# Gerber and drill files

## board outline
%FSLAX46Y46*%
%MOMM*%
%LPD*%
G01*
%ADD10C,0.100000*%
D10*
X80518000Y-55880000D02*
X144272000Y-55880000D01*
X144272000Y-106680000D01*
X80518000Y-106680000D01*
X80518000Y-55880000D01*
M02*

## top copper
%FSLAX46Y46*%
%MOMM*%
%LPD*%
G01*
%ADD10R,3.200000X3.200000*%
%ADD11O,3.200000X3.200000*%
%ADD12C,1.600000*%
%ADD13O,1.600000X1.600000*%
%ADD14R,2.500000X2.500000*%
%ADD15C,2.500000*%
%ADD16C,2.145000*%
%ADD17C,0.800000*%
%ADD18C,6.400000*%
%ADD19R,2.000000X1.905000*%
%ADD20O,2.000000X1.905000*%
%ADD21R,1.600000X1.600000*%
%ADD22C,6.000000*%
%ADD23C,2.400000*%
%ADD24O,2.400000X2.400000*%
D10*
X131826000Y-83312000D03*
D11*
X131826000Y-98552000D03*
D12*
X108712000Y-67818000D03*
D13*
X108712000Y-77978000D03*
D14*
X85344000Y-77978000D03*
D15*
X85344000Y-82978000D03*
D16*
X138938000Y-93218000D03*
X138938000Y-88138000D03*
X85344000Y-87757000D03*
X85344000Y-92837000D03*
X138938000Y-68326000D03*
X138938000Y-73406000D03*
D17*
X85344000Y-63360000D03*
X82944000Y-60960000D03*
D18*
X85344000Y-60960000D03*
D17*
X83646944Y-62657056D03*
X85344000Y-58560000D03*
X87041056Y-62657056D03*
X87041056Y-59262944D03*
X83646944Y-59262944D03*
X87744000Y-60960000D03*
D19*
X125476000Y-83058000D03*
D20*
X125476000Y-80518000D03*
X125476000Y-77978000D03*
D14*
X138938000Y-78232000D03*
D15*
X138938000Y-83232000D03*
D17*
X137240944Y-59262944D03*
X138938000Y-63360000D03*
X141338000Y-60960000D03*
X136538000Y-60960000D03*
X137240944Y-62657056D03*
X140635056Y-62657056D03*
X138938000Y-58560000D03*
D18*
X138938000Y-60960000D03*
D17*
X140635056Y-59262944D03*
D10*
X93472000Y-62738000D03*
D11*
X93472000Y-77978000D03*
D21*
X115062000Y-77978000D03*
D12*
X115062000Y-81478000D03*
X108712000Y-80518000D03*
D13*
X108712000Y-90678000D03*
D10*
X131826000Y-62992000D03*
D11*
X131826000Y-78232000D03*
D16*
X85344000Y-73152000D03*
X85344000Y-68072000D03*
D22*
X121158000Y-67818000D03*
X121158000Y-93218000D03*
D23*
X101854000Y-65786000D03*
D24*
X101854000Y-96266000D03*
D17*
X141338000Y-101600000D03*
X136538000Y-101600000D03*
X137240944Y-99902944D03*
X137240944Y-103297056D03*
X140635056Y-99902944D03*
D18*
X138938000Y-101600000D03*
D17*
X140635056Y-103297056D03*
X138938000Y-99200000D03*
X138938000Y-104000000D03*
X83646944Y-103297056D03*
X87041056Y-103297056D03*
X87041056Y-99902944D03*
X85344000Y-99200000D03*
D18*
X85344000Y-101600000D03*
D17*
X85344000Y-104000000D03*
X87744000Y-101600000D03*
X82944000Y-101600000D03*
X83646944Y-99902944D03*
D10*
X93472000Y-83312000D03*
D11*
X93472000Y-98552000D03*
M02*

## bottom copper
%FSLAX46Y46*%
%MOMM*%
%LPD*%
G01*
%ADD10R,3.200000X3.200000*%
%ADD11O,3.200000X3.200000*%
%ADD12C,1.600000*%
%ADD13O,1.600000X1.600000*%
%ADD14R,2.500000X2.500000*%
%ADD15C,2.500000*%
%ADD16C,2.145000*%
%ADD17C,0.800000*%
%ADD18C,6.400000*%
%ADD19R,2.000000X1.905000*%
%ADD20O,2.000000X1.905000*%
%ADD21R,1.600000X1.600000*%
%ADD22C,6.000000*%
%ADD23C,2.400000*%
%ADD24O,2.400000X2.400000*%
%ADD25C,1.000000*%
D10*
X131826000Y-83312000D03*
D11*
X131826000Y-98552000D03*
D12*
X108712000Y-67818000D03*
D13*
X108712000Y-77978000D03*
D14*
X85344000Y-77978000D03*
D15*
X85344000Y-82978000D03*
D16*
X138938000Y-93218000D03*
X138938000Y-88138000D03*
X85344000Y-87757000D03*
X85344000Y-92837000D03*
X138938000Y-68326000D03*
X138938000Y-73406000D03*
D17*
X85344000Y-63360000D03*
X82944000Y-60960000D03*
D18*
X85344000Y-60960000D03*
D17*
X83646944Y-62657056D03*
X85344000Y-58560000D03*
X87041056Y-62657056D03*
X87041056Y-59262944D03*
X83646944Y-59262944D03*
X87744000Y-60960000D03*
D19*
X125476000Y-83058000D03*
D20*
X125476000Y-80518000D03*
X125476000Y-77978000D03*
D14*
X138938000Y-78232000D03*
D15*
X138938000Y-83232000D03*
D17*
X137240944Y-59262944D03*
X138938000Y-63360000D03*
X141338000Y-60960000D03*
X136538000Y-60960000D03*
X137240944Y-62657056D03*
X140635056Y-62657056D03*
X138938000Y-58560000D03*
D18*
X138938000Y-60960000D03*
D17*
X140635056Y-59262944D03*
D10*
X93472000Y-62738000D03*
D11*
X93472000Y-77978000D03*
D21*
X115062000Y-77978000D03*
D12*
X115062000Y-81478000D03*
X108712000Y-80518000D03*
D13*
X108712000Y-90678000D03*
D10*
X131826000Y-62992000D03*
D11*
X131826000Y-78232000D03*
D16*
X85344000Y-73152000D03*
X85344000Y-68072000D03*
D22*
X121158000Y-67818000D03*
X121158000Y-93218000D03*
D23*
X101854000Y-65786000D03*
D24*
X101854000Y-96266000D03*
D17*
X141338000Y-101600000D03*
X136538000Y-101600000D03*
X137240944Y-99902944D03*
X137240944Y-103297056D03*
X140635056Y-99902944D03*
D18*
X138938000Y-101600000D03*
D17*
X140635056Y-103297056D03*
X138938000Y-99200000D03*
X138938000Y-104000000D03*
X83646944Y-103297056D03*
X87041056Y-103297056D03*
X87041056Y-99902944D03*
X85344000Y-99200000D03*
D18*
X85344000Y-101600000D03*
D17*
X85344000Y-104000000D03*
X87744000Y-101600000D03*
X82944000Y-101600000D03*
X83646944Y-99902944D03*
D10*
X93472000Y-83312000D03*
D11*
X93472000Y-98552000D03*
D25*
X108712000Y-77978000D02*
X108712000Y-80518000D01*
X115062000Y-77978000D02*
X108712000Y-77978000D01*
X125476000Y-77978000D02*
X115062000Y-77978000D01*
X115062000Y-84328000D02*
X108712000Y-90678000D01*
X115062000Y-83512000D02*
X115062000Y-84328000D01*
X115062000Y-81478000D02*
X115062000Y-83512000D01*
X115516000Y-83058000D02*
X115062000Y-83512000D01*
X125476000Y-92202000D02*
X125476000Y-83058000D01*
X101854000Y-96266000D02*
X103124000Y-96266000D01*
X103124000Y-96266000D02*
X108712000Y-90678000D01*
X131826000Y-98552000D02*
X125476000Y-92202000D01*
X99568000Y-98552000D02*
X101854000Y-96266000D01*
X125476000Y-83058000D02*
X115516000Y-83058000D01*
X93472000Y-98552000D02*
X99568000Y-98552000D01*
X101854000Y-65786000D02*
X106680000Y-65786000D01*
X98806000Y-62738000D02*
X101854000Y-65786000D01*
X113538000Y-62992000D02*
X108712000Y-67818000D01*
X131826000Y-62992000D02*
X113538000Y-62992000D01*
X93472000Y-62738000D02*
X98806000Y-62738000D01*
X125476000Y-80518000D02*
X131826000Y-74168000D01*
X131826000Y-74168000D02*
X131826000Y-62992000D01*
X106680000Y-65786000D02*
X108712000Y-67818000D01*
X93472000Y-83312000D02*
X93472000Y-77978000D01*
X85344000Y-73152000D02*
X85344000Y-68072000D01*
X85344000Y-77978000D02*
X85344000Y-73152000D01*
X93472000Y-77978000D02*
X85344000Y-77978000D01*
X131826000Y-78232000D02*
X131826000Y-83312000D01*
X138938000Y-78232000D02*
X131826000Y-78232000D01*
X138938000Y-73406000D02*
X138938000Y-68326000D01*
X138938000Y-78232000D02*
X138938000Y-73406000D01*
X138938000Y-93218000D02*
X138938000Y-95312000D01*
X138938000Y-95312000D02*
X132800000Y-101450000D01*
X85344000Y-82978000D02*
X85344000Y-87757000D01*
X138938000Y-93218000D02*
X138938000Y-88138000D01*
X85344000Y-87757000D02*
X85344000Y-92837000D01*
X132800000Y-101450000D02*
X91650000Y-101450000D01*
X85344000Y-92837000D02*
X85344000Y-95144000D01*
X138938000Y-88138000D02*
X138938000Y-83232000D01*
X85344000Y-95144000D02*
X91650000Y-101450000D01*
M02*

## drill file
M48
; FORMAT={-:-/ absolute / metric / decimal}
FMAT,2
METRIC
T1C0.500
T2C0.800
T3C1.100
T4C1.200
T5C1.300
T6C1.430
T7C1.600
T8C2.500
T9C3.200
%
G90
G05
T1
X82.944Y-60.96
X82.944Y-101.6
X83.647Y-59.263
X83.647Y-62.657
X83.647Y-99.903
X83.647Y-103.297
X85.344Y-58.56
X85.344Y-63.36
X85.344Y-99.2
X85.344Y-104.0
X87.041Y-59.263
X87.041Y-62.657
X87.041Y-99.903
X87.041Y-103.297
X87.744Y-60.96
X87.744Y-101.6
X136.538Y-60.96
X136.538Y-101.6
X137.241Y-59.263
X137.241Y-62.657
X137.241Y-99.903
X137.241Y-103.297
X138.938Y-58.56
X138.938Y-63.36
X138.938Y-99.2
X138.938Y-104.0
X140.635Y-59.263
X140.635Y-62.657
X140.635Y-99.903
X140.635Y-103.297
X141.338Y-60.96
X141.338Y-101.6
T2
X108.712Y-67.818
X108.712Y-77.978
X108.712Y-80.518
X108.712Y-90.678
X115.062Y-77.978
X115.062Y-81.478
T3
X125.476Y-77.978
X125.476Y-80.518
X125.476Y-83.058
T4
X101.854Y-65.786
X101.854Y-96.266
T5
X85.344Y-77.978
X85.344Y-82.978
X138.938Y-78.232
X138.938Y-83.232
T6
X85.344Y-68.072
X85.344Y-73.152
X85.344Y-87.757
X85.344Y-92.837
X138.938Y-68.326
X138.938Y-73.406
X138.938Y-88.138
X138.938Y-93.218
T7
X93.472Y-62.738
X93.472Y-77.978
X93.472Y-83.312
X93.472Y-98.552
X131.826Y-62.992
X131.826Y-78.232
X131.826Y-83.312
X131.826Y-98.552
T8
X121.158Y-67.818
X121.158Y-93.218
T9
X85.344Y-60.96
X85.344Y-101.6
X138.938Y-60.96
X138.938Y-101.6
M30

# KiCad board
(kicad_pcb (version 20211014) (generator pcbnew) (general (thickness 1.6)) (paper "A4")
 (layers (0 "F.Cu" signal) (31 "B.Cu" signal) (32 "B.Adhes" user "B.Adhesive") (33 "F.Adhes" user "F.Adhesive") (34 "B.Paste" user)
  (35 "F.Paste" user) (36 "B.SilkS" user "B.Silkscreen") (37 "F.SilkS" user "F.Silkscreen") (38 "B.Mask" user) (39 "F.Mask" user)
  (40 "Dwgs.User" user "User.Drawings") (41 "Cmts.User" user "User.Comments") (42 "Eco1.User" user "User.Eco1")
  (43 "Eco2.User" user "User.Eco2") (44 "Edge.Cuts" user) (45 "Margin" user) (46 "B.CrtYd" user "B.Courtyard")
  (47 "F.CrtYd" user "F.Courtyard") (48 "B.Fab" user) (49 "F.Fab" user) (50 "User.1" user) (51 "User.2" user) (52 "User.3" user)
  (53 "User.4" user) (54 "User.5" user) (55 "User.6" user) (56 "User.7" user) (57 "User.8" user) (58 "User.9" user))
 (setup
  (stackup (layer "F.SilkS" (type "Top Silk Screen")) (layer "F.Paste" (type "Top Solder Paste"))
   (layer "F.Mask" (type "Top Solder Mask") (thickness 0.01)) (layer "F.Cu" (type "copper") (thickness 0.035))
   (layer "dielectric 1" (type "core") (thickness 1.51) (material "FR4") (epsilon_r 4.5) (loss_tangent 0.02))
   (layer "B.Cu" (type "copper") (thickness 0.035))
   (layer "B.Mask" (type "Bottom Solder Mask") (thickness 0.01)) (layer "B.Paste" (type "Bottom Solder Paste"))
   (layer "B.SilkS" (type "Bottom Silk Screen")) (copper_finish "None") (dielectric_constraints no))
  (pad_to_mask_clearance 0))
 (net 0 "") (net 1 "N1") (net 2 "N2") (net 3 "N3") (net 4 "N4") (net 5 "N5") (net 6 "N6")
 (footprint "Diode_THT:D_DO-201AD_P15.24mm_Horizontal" (layer "F.Cu") (at 131.826 83.312 -90)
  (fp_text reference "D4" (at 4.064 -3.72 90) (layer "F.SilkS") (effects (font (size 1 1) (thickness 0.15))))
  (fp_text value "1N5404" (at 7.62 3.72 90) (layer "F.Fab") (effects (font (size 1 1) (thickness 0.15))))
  (pad "1" thru_hole rect (at 0 0 270) (size 3.2 3.2) (drill 1.6) (layers *.Cu *.Mask) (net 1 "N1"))
  (pad "2" thru_hole oval (at 15.24 0 270) (size 3.2 3.2) (drill 1.6) (layers *.Cu *.Mask) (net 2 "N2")))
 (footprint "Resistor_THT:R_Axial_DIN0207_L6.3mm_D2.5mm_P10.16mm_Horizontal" (layer "F.Cu") (at 108.712 67.818 -90)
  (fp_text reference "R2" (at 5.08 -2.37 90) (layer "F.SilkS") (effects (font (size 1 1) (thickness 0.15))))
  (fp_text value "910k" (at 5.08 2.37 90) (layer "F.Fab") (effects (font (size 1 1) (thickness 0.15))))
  (pad "1" thru_hole circle (at 0 0 270) (size 1.6 1.6) (drill 0.8) (layers *.Cu *.Mask) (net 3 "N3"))
  (pad "2" thru_hole oval (at 10.16 0 270) (size 1.6 1.6) (drill 0.8) (layers *.Cu *.Mask) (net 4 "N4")))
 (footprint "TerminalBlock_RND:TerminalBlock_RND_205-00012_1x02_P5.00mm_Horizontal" (layer "F.Cu") (at 85.344 77.978 -90)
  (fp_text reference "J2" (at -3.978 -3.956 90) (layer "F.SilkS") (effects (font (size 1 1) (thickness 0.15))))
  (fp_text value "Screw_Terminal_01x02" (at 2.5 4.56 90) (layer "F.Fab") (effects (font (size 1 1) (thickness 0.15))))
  (pad "1" thru_hole rect (at 0 0 270) (size 2.5 2.5) (drill 1.3) (layers *.Cu *.Mask) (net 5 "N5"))
  (pad "2" thru_hole circle (at 5 0 270) (size 2.5 2.5) (drill 1.3) (layers *.Cu *.Mask) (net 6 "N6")))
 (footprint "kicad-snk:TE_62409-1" (layer "F.Cu") (at 138.938 90.678 90)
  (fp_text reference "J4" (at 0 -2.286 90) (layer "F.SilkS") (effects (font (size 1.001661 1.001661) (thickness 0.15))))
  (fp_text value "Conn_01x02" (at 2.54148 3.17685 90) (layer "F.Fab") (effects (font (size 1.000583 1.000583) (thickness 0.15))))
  (pad "1" thru_hole circle (at -2.54 0 90) (size 2.145 2.145) (drill 1.43) (layers *.Cu *.Mask) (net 6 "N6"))
  (pad "2" thru_hole circle (at 2.54 0 90) (size 2.145 2.145) (drill 1.43) (layers *.Cu *.Mask) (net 6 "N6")))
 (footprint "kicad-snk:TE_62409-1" (layer "F.Cu") (at 85.344 90.297 -90)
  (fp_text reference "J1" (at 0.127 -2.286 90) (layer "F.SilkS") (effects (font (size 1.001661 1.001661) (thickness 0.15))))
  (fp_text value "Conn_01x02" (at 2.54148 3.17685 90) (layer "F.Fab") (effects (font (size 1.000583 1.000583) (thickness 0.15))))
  (pad "1" thru_hole circle (at -2.54 0 270) (size 2.145 2.145) (drill 1.43) (layers *.Cu *.Mask) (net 6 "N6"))
  (pad "2" thru_hole circle (at 2.54 0 270) (size 2.145 2.145) (drill 1.43) (layers *.Cu *.Mask) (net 6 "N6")))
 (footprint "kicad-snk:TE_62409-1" (layer "F.Cu") (at 138.938 70.866 -90)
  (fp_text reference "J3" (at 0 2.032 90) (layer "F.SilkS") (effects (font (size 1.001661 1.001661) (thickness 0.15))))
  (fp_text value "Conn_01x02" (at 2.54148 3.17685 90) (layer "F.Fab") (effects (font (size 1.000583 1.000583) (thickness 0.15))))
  (pad "1" thru_hole circle (at -2.54 0 270) (size 2.145 2.145) (drill 1.43) (layers *.Cu *.Mask) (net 1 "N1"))
  (pad "2" thru_hole circle (at 2.54 0 270) (size 2.145 2.145) (drill 1.43) (layers *.Cu *.Mask) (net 1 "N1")))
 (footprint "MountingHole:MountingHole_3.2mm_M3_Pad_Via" (layer "F.Cu") (at 85.344 60.96)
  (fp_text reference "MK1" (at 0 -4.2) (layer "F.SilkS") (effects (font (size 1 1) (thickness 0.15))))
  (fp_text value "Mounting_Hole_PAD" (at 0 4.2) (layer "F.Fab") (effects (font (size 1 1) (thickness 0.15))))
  (pad "1" thru_hole circle (at 0 2.4) (size 0.8 0.8) (drill 0.5) (layers *.Cu *.Mask))
  (pad "1" thru_hole circle (at -2.4 0) (size 0.8 0.8) (drill 0.5) (layers *.Cu *.Mask))
  (pad "1" thru_hole circle (at 0 0) (size 6.4 6.4) (drill 3.2) (layers *.Cu *.Mask))
  (pad "1" thru_hole circle (at -1.697056 1.697056) (size 0.8 0.8) (drill 0.5) (layers *.Cu *.Mask))
  (pad "1" thru_hole circle (at 0 -2.4) (size 0.8 0.8) (drill 0.5) (layers *.Cu *.Mask))
  (pad "1" thru_hole circle (at 1.697056 1.697056) (size 0.8 0.8) (drill 0.5) (layers *.Cu *.Mask))
  (pad "1" thru_hole circle (at 1.697056 -1.697056) (size 0.8 0.8) (drill 0.5) (layers *.Cu *.Mask))
  (pad "1" thru_hole circle (at -1.697056 -1.697056) (size 0.8 0.8) (drill 0.5) (layers *.Cu *.Mask))
  (pad "1" thru_hole circle (at 2.4 0) (size 0.8 0.8) (drill 0.5) (layers *.Cu *.Mask)))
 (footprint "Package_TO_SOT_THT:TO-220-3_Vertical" (layer "F.Cu") (at 125.476 83.058 90)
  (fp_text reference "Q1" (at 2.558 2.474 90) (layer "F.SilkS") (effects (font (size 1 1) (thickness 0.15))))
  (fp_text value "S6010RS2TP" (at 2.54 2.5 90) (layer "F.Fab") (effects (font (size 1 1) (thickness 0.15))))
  (pad "1" thru_hole rect (at 0 0 90) (size 1.905 2) (drill 1.1) (layers *.Cu *.Mask) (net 2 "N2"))
  (pad "2" thru_hole oval (at 2.54 0 90) (size 1.905 2) (drill 1.1) (layers *.Cu *.Mask) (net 3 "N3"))
  (pad "3" thru_hole oval (at 5.08 0 90) (size 1.905 2) (drill 1.1) (layers *.Cu *.Mask) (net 4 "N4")))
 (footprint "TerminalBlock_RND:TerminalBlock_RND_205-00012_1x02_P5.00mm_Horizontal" (layer "F.Cu") (at 138.938 78.232 -90)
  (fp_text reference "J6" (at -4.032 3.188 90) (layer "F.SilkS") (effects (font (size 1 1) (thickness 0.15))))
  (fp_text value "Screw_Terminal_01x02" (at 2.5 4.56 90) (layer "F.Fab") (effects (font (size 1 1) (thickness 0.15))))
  (pad "1" thru_hole rect (at 0 0 270) (size 2.5 2.5) (drill 1.3) (layers *.Cu *.Mask) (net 1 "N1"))
  (pad "2" thru_hole circle (at 5 0 270) (size 2.5 2.5) (drill 1.3) (layers *.Cu *.Mask) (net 6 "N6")))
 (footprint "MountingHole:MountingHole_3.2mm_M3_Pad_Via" (layer "F.Cu") (at 138.938 60.96)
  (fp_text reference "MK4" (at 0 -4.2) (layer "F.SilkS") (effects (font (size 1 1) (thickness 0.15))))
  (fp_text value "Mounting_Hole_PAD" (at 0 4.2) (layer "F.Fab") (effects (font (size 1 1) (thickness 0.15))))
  (pad "1" thru_hole circle (at -1.697056 -1.697056) (size 0.8 0.8) (drill 0.5) (layers *.Cu *.Mask))
  (pad "1" thru_hole circle (at 0 2.4) (size 0.8 0.8) (drill 0.5) (layers *.Cu *.Mask))
  (pad "1" thru_hole circle (at 2.4 0) (size 0.8 0.8) (drill 0.5) (layers *.Cu *.Mask))
  (pad "1" thru_hole circle (at -2.4 0) (size 0.8 0.8) (drill 0.5) (layers *.Cu *.Mask))
  (pad "1" thru_hole circle (at -1.697056 1.697056) (size 0.8 0.8) (drill 0.5) (layers *.Cu *.Mask))
  (pad "1" thru_hole circle (at 1.697056 1.697056) (size 0.8 0.8) (drill 0.5) (layers *.Cu *.Mask))
  (pad "1" thru_hole circle (at 0 -2.4) (size 0.8 0.8) (drill 0.5) (layers *.Cu *.Mask))
  (pad "1" thru_hole circle (at 0 0) (size 6.4 6.4) (drill 3.2) (layers *.Cu *.Mask))
  (pad "1" thru_hole circle (at 1.697056 -1.697056) (size 0.8 0.8) (drill 0.5) (layers *.Cu *.Mask)))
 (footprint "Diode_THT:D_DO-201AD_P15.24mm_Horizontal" (layer "F.Cu") (at 93.472 62.738 -90)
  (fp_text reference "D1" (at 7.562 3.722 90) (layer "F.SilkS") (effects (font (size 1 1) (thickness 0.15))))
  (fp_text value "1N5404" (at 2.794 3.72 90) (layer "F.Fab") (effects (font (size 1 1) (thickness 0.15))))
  (pad "1" thru_hole rect (at 0 0 270) (size 3.2 3.2) (drill 1.6) (layers *.Cu *.Mask) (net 3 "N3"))
  (pad "2" thru_hole oval (at 15.24 0 270) (size 3.2 3.2) (drill 1.6) (layers *.Cu *.Mask) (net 5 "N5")))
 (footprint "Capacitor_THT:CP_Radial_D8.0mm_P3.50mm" (layer "F.Cu") (at 115.062 77.978 -90)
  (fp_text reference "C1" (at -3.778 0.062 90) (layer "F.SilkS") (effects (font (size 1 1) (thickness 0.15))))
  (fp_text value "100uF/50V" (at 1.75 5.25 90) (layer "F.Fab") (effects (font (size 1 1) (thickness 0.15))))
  (pad "1" thru_hole rect (at 0 0 270) (size 1.6 1.6) (drill 0.8) (layers *.Cu *.Mask) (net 4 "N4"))
  (pad "2" thru_hole circle (at 3.5 0 270) (size 1.6 1.6) (drill 0.8) (layers *.Cu *.Mask) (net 2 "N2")))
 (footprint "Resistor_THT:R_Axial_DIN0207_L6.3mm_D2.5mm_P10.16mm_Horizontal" (layer "F.Cu") (at 108.712 80.518 -90)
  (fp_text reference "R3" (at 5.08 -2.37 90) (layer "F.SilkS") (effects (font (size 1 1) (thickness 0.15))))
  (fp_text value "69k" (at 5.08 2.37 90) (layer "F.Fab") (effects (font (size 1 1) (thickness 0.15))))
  (pad "1" thru_hole circle (at 0 0 270) (size 1.6 1.6) (drill 0.8) (layers *.Cu *.Mask) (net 4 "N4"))
  (pad "2" thru_hole oval (at 10.16 0 270) (size 1.6 1.6) (drill 0.8) (layers *.Cu *.Mask) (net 2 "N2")))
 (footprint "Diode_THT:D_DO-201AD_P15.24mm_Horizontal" (layer "F.Cu") (at 131.826 62.992 -90)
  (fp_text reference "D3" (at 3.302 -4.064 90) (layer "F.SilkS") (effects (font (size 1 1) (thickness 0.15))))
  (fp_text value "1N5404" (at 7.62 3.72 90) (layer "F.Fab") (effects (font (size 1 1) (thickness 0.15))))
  (pad "1" thru_hole rect (at 0 0 270) (size 3.2 3.2) (drill 1.6) (layers *.Cu *.Mask) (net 3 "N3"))
  (pad "2" thru_hole oval (at 15.24 0 270) (size 3.2 3.2) (drill 1.6) (layers *.Cu *.Mask) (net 1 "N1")))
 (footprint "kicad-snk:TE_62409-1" (layer "F.Cu") (at 85.344 70.612 90)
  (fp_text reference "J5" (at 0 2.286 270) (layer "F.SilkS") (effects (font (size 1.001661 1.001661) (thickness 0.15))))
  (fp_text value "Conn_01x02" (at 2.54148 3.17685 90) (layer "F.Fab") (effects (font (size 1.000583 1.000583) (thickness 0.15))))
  (pad "1" thru_hole circle (at -2.54 0 90) (size 2.145 2.145) (drill 1.43) (layers *.Cu *.Mask) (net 5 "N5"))
  (pad "2" thru_hole circle (at 2.54 0 90) (size 2.145 2.145) (drill 1.43) (layers *.Cu *.Mask) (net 5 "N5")))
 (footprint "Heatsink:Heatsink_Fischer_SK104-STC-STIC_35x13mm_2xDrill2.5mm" (layer "F.Cu") (at 121.158 80.518 90)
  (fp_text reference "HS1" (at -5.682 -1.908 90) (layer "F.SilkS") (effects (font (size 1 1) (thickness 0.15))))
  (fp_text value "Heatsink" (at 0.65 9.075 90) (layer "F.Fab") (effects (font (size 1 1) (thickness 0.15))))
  (pad "1" thru_hole circle (at 12.7 0 90) (size 6 6) (drill 2.5) (layers *.Cu *.Mask))
  (pad "1" thru_hole circle (at -12.7 0 270) (size 6 6) (drill 2.5) (layers *.Cu *.Mask)))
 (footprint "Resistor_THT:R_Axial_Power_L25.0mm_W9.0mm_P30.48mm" (layer "F.Cu") (at 101.854 65.786 -90)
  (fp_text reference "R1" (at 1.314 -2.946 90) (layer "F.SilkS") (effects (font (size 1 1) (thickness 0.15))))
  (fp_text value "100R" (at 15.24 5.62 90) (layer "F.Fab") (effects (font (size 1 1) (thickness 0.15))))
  (pad "1" thru_hole circle (at 0 0 270) (size 2.4 2.4) (drill 1.2) (layers *.Cu *.Mask) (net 3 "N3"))
  (pad "2" thru_hole oval (at 30.48 0 270) (size 2.4 2.4) (drill 1.2) (layers *.Cu *.Mask) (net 2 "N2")))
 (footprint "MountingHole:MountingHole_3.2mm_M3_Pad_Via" (layer "F.Cu") (at 138.938 101.6)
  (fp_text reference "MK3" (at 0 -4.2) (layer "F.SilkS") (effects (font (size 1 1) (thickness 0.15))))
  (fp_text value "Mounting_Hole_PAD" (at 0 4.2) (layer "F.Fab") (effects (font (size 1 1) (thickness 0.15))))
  (pad "1" thru_hole circle (at 2.4 0) (size 0.8 0.8) (drill 0.5) (layers *.Cu *.Mask))
  (pad "1" thru_hole circle (at -2.4 0) (size 0.8 0.8) (drill 0.5) (layers *.Cu *.Mask))
  (pad "1" thru_hole circle (at -1.697056 -1.697056) (size 0.8 0.8) (drill 0.5) (layers *.Cu *.Mask))
  (pad "1" thru_hole circle (at -1.697056 1.697056) (size 0.8 0.8) (drill 0.5) (layers *.Cu *.Mask))
  (pad "1" thru_hole circle (at 1.697056 -1.697056) (size 0.8 0.8) (drill 0.5) (layers *.Cu *.Mask))
  (pad "1" thru_hole circle (at 0 0) (size 6.4 6.4) (drill 3.2) (layers *.Cu *.Mask))
  (pad "1" thru_hole circle (at 1.697056 1.697056) (size 0.8 0.8) (drill 0.5) (layers *.Cu *.Mask))
  (pad "1" thru_hole circle (at 0 -2.4) (size 0.8 0.8) (drill 0.5) (layers *.Cu *.Mask))
  (pad "1" thru_hole circle (at 0 2.4) (size 0.8 0.8) (drill 0.5) (layers *.Cu *.Mask)))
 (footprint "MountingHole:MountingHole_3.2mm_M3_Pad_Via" (layer "F.Cu") (at 85.344 101.6)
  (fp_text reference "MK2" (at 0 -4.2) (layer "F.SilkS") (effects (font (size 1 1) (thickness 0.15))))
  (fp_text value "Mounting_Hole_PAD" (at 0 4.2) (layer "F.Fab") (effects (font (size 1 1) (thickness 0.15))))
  (pad "1" thru_hole circle (at -1.697056 1.697056) (size 0.8 0.8) (drill 0.5) (layers *.Cu *.Mask))
  (pad "1" thru_hole circle (at 1.697056 1.697056) (size 0.8 0.8) (drill 0.5) (layers *.Cu *.Mask))
  (pad "1" thru_hole circle (at 1.697056 -1.697056) (size 0.8 0.8) (drill 0.5) (layers *.Cu *.Mask))
  (pad "1" thru_hole circle (at 0 -2.4) (size 0.8 0.8) (drill 0.5) (layers *.Cu *.Mask))
  (pad "1" thru_hole circle (at 0 0) (size 6.4 6.4) (drill 3.2) (layers *.Cu *.Mask))
  (pad "1" thru_hole circle (at 0 2.4) (size 0.8 0.8) (drill 0.5) (layers *.Cu *.Mask))
  (pad "1" thru_hole circle (at 2.4 0) (size 0.8 0.8) (drill 0.5) (layers *.Cu *.Mask))
  (pad "1" thru_hole circle (at -2.4 0) (size 0.8 0.8) (drill 0.5) (layers *.Cu *.Mask))
  (pad "1" thru_hole circle (at -1.697056 -1.697056) (size 0.8 0.8) (drill 0.5) (layers *.Cu *.Mask)))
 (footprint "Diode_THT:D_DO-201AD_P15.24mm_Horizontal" (layer "F.Cu") (at 93.472 83.312 -90)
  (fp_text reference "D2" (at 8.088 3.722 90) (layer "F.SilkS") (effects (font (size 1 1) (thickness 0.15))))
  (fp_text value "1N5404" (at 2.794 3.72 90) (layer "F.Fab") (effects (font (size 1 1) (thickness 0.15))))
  (pad "1" thru_hole rect (at 0 0 270) (size 3.2 3.2) (drill 1.6) (layers *.Cu *.Mask) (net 5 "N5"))
  (pad "2" thru_hole oval (at 15.24 0 270) (size 3.2 3.2) (drill 1.6) (layers *.Cu *.Mask) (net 2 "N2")))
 (gr_rect (start 80.518 55.88) (end 144.272 106.68) (layer "Edge.Cuts") (width 0.1) (fill none))
 (segment (start 108.712 77.978) (end 108.712 80.518) (width 1) (layer "B.Cu") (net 4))
 (segment (start 115.062 77.978) (end 108.712 77.978) (width 1) (layer "B.Cu") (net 4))
 (segment (start 125.476 77.978) (end 115.062 77.978) (width 1) (layer "B.Cu") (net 4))
 (segment (start 115.062 84.328) (end 108.712 90.678) (width 1) (layer "B.Cu") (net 2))
 (segment (start 115.062 83.512) (end 115.062 84.328) (width 1) (layer "B.Cu") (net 2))
 (segment (start 115.062 81.478) (end 115.062 83.512) (width 1) (layer "B.Cu") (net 2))
 (segment (start 115.516 83.058) (end 115.062 83.512) (width 1) (layer "B.Cu") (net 2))
 (segment (start 125.476 92.202) (end 125.476 83.058) (width 1) (layer "B.Cu") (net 2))
 (segment (start 101.854 96.266) (end 103.124 96.266) (width 1) (layer "B.Cu") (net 2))
 (segment (start 103.124 96.266) (end 108.712 90.678) (width 1) (layer "B.Cu") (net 2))
 (segment (start 131.826 98.552) (end 125.476 92.202) (width 1) (layer "B.Cu") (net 2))
 (segment (start 99.568 98.552) (end 101.854 96.266) (width 1) (layer "B.Cu") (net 2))
 (segment (start 125.476 83.058) (end 115.516 83.058) (width 1) (layer "B.Cu") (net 2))
 (segment (start 93.472 98.552) (end 99.568 98.552) (width 1) (layer "B.Cu") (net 2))
 (segment (start 101.854 65.786) (end 106.68 65.786) (width 1) (layer "B.Cu") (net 3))
 (segment (start 98.806 62.738) (end 101.854 65.786) (width 1) (layer "B.Cu") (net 3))
 (segment (start 113.538 62.992) (end 108.712 67.818) (width 1) (layer "B.Cu") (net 3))
 (segment (start 131.826 62.992) (end 113.538 62.992) (width 1) (layer "B.Cu") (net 3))
 (segment (start 93.472 62.738) (end 98.806 62.738) (width 1) (layer "B.Cu") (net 3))
 (segment (start 125.476 80.518) (end 131.826 74.168) (width 1) (layer "B.Cu") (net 3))
 (segment (start 131.826 74.168) (end 131.826 62.992) (width 1) (layer "B.Cu") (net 3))
 (segment (start 106.68 65.786) (end 108.712 67.818) (width 1) (layer "B.Cu") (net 3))
 (segment (start 93.472 83.312) (end 93.472 77.978) (width 1) (layer "B.Cu") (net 5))
 (segment (start 85.344 73.152) (end 85.344 68.072) (width 1) (layer "B.Cu") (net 5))
 (segment (start 85.344 77.978) (end 85.344 73.152) (width 1) (layer "B.Cu") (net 5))
 (segment (start 93.472 77.978) (end 85.344 77.978) (width 1) (layer "B.Cu") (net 5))
 (segment (start 131.826 78.232) (end 131.826 83.312) (width 1) (layer "B.Cu") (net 1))
 (segment (start 138.938 78.232) (end 131.826 78.232) (width 1) (layer "B.Cu") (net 1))
 (segment (start 138.938 73.406) (end 138.938 68.326) (width 1) (layer "B.Cu") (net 1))
 (segment (start 138.938 78.232) (end 138.938 73.406) (width 1) (layer "B.Cu") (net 1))
 (segment (start 138.938 93.218) (end 138.938 95.312) (width 1) (layer "B.Cu") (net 6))
 (segment (start 138.938 95.312) (end 132.8 101.45) (width 1) (layer "B.Cu") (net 6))
 (segment (start 85.344 82.978) (end 85.344 87.757) (width 1) (layer "B.Cu") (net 6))
 (segment (start 138.938 93.218) (end 138.938 88.138) (width 1) (layer "B.Cu") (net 6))
 (segment (start 85.344 87.757) (end 85.344 92.837) (width 1) (layer "B.Cu") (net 6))
 (segment (start 132.8 101.45) (end 91.65 101.45) (width 1) (layer "B.Cu") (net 6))
 (segment (start 85.344 92.837) (end 85.344 95.144) (width 1) (layer "B.Cu") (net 6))
 (segment (start 138.938 88.138) (end 138.938 83.232) (width 1) (layer "B.Cu") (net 6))
 (segment (start 85.344 95.144) (end 91.65 101.45) (width 1) (layer "B.Cu") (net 6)))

